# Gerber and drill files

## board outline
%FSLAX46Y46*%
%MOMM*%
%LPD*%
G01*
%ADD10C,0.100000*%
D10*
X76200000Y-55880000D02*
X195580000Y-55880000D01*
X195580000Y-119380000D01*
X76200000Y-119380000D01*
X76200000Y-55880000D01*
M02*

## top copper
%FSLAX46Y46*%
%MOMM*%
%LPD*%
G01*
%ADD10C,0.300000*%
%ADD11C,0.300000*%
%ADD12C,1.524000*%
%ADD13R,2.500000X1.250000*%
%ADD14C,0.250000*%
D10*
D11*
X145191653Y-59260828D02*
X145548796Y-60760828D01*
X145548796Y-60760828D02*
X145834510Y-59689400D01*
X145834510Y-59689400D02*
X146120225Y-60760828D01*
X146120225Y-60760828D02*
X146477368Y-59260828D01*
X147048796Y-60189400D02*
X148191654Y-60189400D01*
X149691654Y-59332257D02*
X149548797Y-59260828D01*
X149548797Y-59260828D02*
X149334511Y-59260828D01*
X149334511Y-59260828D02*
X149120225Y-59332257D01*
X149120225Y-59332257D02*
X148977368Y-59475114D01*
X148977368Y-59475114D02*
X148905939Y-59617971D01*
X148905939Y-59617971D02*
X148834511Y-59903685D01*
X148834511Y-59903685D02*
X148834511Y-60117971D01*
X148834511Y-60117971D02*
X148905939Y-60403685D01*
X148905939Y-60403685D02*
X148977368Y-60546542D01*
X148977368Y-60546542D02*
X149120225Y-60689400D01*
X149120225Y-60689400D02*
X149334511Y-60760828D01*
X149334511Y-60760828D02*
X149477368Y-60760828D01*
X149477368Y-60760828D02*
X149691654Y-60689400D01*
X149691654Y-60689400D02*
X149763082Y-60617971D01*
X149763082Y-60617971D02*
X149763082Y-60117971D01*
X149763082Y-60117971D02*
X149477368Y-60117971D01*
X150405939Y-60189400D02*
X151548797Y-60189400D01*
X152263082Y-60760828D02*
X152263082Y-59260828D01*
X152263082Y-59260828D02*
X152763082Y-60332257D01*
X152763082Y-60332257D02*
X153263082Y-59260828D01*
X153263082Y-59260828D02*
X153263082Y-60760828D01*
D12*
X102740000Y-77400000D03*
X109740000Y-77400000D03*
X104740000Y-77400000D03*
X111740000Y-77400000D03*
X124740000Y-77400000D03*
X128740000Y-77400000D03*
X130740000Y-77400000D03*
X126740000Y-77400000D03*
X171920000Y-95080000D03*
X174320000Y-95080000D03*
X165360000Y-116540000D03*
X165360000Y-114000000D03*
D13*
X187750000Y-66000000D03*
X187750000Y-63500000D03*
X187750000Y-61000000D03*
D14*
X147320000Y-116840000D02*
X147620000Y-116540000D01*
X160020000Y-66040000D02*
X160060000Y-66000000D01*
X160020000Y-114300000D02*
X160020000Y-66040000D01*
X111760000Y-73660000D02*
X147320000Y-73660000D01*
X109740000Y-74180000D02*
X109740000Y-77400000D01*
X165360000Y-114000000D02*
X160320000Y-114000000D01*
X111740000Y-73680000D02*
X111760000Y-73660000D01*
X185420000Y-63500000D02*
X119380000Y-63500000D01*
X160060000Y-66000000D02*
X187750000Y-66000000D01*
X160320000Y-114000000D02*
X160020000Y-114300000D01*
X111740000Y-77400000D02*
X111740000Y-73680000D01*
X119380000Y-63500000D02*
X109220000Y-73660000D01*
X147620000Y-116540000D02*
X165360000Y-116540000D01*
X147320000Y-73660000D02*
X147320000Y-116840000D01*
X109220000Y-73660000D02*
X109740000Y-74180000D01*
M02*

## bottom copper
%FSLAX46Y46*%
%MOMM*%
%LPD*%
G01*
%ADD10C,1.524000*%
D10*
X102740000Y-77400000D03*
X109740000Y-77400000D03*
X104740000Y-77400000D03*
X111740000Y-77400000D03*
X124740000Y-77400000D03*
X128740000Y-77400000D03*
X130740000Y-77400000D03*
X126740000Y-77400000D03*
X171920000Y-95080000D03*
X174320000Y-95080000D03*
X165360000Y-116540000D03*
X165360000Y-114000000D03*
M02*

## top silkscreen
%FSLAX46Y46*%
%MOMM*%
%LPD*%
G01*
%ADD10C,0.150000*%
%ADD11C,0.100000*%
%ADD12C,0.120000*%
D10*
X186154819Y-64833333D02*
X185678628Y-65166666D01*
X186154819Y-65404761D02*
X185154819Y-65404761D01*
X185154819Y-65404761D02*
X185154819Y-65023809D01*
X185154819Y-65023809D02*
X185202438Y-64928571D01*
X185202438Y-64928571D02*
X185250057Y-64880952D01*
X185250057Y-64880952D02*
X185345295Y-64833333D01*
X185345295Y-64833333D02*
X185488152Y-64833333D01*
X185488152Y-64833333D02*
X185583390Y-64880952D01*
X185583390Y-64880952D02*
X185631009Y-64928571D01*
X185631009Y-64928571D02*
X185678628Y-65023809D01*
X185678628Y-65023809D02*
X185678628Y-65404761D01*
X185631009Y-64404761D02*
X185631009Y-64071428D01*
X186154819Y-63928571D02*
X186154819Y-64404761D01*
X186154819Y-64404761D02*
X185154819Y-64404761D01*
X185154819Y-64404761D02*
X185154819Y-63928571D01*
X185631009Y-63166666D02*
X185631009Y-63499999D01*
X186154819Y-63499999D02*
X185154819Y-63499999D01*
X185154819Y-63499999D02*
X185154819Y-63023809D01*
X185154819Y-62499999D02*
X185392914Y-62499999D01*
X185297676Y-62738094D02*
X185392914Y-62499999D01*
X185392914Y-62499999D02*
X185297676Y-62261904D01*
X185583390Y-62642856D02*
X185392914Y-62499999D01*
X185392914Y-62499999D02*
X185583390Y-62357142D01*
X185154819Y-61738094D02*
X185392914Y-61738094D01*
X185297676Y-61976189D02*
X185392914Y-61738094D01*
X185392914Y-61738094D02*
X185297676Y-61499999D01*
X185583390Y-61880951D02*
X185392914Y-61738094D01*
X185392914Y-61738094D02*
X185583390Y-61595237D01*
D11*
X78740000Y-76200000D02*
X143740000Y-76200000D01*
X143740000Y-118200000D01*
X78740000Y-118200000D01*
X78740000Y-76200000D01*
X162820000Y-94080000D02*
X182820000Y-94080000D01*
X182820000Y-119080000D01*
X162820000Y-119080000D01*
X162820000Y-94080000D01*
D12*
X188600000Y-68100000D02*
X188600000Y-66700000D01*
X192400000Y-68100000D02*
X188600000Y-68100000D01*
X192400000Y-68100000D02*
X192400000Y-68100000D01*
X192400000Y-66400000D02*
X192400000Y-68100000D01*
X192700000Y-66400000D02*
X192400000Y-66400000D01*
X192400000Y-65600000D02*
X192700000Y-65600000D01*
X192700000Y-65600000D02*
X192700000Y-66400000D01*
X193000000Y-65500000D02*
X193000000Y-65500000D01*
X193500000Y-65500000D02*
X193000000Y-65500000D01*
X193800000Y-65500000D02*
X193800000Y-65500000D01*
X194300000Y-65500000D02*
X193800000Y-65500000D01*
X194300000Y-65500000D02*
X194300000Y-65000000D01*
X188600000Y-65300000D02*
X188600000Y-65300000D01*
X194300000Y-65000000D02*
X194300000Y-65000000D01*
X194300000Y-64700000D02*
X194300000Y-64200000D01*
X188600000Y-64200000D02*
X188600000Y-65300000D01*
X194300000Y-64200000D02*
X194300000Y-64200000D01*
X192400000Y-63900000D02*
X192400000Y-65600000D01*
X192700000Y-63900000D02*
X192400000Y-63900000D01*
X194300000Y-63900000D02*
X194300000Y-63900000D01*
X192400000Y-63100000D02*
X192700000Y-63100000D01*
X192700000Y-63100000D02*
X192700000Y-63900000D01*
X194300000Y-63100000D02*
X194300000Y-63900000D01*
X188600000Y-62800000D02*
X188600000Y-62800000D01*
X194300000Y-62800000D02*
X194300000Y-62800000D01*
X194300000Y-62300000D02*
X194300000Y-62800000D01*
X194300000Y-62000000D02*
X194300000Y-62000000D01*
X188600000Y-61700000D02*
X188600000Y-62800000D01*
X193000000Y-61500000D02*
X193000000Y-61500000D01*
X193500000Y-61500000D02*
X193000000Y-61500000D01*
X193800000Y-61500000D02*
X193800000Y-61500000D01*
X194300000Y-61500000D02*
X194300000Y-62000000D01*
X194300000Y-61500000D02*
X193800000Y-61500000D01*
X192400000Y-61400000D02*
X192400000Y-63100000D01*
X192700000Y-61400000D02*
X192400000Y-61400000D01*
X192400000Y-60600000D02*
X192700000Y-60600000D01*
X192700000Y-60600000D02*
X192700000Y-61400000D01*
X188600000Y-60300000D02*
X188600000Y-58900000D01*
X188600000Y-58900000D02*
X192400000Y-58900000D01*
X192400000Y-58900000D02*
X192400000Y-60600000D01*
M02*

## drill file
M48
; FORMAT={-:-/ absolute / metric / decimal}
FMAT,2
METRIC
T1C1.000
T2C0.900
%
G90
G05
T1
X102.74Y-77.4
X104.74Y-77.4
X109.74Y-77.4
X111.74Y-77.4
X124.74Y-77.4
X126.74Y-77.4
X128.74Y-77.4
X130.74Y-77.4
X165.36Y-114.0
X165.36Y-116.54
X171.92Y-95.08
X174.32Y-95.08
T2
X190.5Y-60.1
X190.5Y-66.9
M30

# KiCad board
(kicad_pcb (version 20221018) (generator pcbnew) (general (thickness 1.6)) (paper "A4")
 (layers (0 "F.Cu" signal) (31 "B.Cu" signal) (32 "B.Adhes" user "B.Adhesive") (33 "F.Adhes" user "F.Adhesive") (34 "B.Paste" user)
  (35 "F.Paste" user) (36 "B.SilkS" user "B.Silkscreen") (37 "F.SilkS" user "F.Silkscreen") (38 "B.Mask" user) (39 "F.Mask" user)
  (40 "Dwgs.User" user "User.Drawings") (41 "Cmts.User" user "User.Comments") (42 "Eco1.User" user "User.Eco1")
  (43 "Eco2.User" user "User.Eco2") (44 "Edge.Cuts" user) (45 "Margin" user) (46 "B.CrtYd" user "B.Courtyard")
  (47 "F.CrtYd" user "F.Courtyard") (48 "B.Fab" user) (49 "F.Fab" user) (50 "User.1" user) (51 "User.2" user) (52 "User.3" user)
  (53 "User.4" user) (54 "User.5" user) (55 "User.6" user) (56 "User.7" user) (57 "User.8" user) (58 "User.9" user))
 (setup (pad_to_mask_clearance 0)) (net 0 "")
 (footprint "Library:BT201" (layer "F.Cu") (at 78.74 76.2)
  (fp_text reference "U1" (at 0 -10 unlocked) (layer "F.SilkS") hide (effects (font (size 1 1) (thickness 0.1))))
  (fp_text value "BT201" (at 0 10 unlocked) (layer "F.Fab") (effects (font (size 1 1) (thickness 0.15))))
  (fp_rect (start 0 0) (end 65 42) (stroke (width 0.1) (type default)) (fill none) (layer "F.SilkS"))
  (pad "1" thru_hole circle (at 24 1.2) (size 1.524 1.524) (drill 1) (layers "*.Cu" "*.Mask"))
  (pad "1" thru_hole circle (at 31 1.2) (size 1.524 1.524) (drill 1) (layers "*.Cu" "*.Mask"))
  (pad "2" thru_hole circle (at 26 1.2) (size 1.524 1.524) (drill 1) (layers "*.Cu" "*.Mask"))
  (pad "2" thru_hole circle (at 33 1.2) (size 1.524 1.524) (drill 1) (layers "*.Cu" "*.Mask"))
  (pad "5" thru_hole circle (at 46 1.2) (size 1.524 1.524) (drill 1) (layers "*.Cu" "*.Mask"))
  (pad "6" thru_hole circle (at 50 1.2) (size 1.524 1.524) (drill 1) (layers "*.Cu" "*.Mask"))
  (pad "7" thru_hole circle (at 52 1.2) (size 1.524 1.524) (drill 1) (layers "*.Cu" "*.Mask"))
  (pad "9" thru_hole circle (at 48 1.2) (size 1.524 1.524) (drill 1) (layers "*.Cu" "*.Mask")))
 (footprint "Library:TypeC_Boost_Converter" (layer "F.Cu") (at 162.82 119.08 90)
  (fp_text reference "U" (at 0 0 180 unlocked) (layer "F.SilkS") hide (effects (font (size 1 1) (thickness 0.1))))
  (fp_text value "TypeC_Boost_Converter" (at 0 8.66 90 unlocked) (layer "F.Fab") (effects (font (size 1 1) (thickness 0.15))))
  (fp_rect (start 25 20) (end 0 0) (stroke (width 0.1) (type default)) (fill none) (layer "F.SilkS"))
  (pad "1" thru_hole circle (at 24 9.1 90) (size 1.524 1.524) (drill 1) (layers "*.Cu" "*.Mask"))
  (pad "2" thru_hole circle (at 24 11.5 90) (size 1.524 1.524) (drill 1) (layers "*.Cu" "*.Mask"))
  (pad "3" thru_hole circle (at 2.54 2.54 90) (size 1.524 1.524) (drill 1) (layers "*.Cu" "*.Mask"))
  (pad "4" thru_hole circle (at 5.08 2.54 90) (size 1.524 1.524) (drill 1) (layers "*.Cu" "*.Mask")))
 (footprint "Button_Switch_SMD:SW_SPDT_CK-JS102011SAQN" (layer "F.Cu") (at 190.5 63.5 90)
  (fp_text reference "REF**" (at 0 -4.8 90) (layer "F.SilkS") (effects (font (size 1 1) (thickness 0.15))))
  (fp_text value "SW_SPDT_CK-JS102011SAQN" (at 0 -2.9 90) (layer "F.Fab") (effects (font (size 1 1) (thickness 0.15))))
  (fp_line (start -4.6 -1.9) (end -3.2 -1.9) (stroke (width 0.12) (type solid)) (layer "F.SilkS"))
  (fp_line (start -4.6 1.9) (end -4.6 -1.9) (stroke (width 0.12) (type solid)) (layer "F.SilkS"))
  (fp_line (start -4.6 1.9) (end -4.6 1.9) (stroke (width 0.12) (type solid)) (layer "F.SilkS"))
  (fp_line (start -2.9 1.9) (end -4.6 1.9) (stroke (width 0.12) (type solid)) (layer "F.SilkS"))
  (fp_line (start -2.9 2.2) (end -2.9 1.9) (stroke (width 0.12) (type solid)) (layer "F.SilkS"))
  (fp_line (start -2.1 1.9) (end -2.1 2.2) (stroke (width 0.12) (type solid)) (layer "F.SilkS"))
  (fp_line (start -2.1 2.2) (end -2.9 2.2) (stroke (width 0.12) (type solid)) (layer "F.SilkS"))
  (fp_line (start -2 2.5) (end -2 2.5) (stroke (width 0.12) (type solid)) (layer "F.SilkS"))
  (fp_line (start -2 3) (end -2 2.5) (stroke (width 0.12) (type solid)) (layer "F.SilkS"))
  (fp_line (start -2 3.3) (end -2 3.3) (stroke (width 0.12) (type solid)) (layer "F.SilkS"))
  (fp_line (start -2 3.8) (end -2 3.3) (stroke (width 0.12) (type solid)) (layer "F.SilkS"))
  (fp_line (start -2 3.8) (end -1.5 3.8) (stroke (width 0.12) (type solid)) (layer "F.SilkS"))
  (fp_line (start -1.8 -1.9) (end -1.8 -1.9) (stroke (width 0.12) (type solid)) (layer "F.SilkS"))
  (fp_line (start -1.5 3.8) (end -1.5 3.8) (stroke (width 0.12) (type solid)) (layer "F.SilkS"))
  (fp_line (start -1.2 3.8) (end -0.7 3.8) (stroke (width 0.12) (type solid)) (layer "F.SilkS"))
  (fp_line (start -0.7 -1.9) (end -1.8 -1.9) (stroke (width 0.12) (type solid)) (layer "F.SilkS"))
  (fp_line (start -0.7 3.8) (end -0.7 3.8) (stroke (width 0.12) (type solid)) (layer "F.SilkS"))
  (fp_line (start -0.4 1.9) (end -2.1 1.9) (stroke (width 0.12) (type solid)) (layer "F.SilkS"))
  (fp_line (start -0.4 2.2) (end -0.4 1.9) (stroke (width 0.12) (type solid)) (layer "F.SilkS"))
  (fp_line (start -0.4 3.8) (end -0.4 3.8) (stroke (width 0.12) (type solid)) (layer "F.SilkS"))
  (fp_line (start 0.4 1.9) (end 0.4 2.2) (stroke (width 0.12) (type solid)) (layer "F.SilkS"))
  (fp_line (start 0.4 2.2) (end -0.4 2.2) (stroke (width 0.12) (type solid)) (layer "F.SilkS"))
  (fp_line (start 0.4 3.8) (end -0.4 3.8) (stroke (width 0.12) (type solid)) (layer "F.SilkS"))
  (fp_line (start 0.7 -1.9) (end 0.7 -1.9) (stroke (width 0.12) (type solid)) (layer "F.SilkS"))
  (fp_line (start 0.7 3.8) (end 0.7 3.8) (stroke (width 0.12) (type solid)) (layer "F.SilkS"))
  (fp_line (start 1.2 3.8) (end 0.7 3.8) (stroke (width 0.12) (type solid)) (layer "F.SilkS"))
  (fp_line (start 1.5 3.8) (end 1.5 3.8) (stroke (width 0.12) (type solid)) (layer "F.SilkS"))
  (fp_line (start 1.8 -1.9) (end 0.7 -1.9) (stroke (width 0.12) (type solid)) (layer "F.SilkS"))
  (fp_line (start 2 2.5) (end 2 2.5) (stroke (width 0.12) (type solid)) (layer "F.SilkS"))
  (fp_line (start 2 3) (end 2 2.5) (stroke (width 0.12) (type solid)) (layer "F.SilkS"))
  (fp_line (start 2 3.3) (end 2 3.3) (stroke (width 0.12) (type solid)) (layer "F.SilkS"))
  (fp_line (start 2 3.8) (end 1.5 3.8) (stroke (width 0.12) (type solid)) (layer "F.SilkS"))
  (fp_line (start 2 3.8) (end 2 3.3) (stroke (width 0.12) (type solid)) (layer "F.SilkS"))
  (fp_line (start 2.1 1.9) (end 0.4 1.9) (stroke (width 0.12) (type solid)) (layer "F.SilkS"))
  (fp_line (start 2.1 2.2) (end 2.1 1.9) (stroke (width 0.12) (type solid)) (layer "F.SilkS"))
  (fp_line (start 2.9 1.9) (end 2.9 2.2) (stroke (width 0.12) (type solid)) (layer "F.SilkS"))
  (fp_line (start 2.9 2.2) (end 2.1 2.2) (stroke (width 0.12) (type solid)) (layer "F.SilkS"))
  (fp_line (start 3.2 -1.9) (end 4.6 -1.9) (stroke (width 0.12) (type solid)) (layer "F.SilkS"))
  (fp_line (start 4.6 -1.9) (end 4.6 1.9) (stroke (width 0.12) (type solid)) (layer "F.SilkS"))
  (fp_line (start 4.6 1.9) (end 2.9 1.9) (stroke (width 0.12) (type solid)) (layer "F.SilkS"))
  (pad "" np_thru_hole circle (at -3.4 0 90) (size 0.9 0.9) (drill 0.9) (layers "*.Cu" "*.Mask"))
  (pad "" np_thru_hole circle (at 3.4 0 90) (size 0.9 0.9) (drill 0.9) (layers "*.Cu" "*.Mask"))
  (pad "1" smd rect (at -2.5 -2.75 90) (size 1.25 2.5) (layers "F.Cu" "F.Paste" "F.Mask"))
  (pad "2" smd rect (at 0 -2.75 90) (size 1.25 2.5) (layers "F.Cu" "F.Paste" "F.Mask"))
  (pad "3" smd rect (at 2.5 -2.75 90) (size 1.25 2.5) (layers "F.Cu" "F.Paste" "F.Mask")))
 (gr_rect (start 76.2 55.88) (end 195.58 119.38) (stroke (width 0.1) (type default)) (fill none) (layer "Edge.Cuts"))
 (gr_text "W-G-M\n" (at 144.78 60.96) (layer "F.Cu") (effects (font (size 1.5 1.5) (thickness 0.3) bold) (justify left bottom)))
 (segment (start 147.32 116.84) (end 147.62 116.54) (width 0.25) (layer "F.Cu") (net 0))
 (segment (start 160.02 66.04) (end 160.06 66) (width 0.25) (layer "F.Cu") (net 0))
 (segment (start 160.02 114.3) (end 160.02 66.04) (width 0.25) (layer "F.Cu") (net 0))
 (segment (start 111.76 73.66) (end 147.32 73.66) (width 0.25) (layer "F.Cu") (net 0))
 (segment (start 109.74 74.18) (end 109.74 77.4) (width 0.25) (layer "F.Cu") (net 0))
 (segment (start 165.36 114) (end 160.32 114) (width 0.25) (layer "F.Cu") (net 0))
 (segment (start 111.74 73.68) (end 111.76 73.66) (width 0.25) (layer "F.Cu") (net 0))
 (segment (start 185.42 63.5) (end 119.38 63.5) (width 0.25) (layer "F.Cu") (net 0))
 (segment (start 160.06 66) (end 187.75 66) (width 0.25) (layer "F.Cu") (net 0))
 (segment (start 160.32 114) (end 160.02 114.3) (width 0.25) (layer "F.Cu") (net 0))
 (segment (start 111.74 77.4) (end 111.74 73.68) (width 0.25) (layer "F.Cu") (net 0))
 (segment (start 119.38 63.5) (end 109.22 73.66) (width 0.25) (layer "F.Cu") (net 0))
 (segment (start 147.62 116.54) (end 165.36 116.54) (width 0.25) (layer "F.Cu") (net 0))
 (segment (start 147.32 73.66) (end 147.32 116.84) (width 0.25) (layer "F.Cu") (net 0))
 (segment (start 109.22 73.66) (end 109.74 74.18) (width 0.25) (layer "F.Cu") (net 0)))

